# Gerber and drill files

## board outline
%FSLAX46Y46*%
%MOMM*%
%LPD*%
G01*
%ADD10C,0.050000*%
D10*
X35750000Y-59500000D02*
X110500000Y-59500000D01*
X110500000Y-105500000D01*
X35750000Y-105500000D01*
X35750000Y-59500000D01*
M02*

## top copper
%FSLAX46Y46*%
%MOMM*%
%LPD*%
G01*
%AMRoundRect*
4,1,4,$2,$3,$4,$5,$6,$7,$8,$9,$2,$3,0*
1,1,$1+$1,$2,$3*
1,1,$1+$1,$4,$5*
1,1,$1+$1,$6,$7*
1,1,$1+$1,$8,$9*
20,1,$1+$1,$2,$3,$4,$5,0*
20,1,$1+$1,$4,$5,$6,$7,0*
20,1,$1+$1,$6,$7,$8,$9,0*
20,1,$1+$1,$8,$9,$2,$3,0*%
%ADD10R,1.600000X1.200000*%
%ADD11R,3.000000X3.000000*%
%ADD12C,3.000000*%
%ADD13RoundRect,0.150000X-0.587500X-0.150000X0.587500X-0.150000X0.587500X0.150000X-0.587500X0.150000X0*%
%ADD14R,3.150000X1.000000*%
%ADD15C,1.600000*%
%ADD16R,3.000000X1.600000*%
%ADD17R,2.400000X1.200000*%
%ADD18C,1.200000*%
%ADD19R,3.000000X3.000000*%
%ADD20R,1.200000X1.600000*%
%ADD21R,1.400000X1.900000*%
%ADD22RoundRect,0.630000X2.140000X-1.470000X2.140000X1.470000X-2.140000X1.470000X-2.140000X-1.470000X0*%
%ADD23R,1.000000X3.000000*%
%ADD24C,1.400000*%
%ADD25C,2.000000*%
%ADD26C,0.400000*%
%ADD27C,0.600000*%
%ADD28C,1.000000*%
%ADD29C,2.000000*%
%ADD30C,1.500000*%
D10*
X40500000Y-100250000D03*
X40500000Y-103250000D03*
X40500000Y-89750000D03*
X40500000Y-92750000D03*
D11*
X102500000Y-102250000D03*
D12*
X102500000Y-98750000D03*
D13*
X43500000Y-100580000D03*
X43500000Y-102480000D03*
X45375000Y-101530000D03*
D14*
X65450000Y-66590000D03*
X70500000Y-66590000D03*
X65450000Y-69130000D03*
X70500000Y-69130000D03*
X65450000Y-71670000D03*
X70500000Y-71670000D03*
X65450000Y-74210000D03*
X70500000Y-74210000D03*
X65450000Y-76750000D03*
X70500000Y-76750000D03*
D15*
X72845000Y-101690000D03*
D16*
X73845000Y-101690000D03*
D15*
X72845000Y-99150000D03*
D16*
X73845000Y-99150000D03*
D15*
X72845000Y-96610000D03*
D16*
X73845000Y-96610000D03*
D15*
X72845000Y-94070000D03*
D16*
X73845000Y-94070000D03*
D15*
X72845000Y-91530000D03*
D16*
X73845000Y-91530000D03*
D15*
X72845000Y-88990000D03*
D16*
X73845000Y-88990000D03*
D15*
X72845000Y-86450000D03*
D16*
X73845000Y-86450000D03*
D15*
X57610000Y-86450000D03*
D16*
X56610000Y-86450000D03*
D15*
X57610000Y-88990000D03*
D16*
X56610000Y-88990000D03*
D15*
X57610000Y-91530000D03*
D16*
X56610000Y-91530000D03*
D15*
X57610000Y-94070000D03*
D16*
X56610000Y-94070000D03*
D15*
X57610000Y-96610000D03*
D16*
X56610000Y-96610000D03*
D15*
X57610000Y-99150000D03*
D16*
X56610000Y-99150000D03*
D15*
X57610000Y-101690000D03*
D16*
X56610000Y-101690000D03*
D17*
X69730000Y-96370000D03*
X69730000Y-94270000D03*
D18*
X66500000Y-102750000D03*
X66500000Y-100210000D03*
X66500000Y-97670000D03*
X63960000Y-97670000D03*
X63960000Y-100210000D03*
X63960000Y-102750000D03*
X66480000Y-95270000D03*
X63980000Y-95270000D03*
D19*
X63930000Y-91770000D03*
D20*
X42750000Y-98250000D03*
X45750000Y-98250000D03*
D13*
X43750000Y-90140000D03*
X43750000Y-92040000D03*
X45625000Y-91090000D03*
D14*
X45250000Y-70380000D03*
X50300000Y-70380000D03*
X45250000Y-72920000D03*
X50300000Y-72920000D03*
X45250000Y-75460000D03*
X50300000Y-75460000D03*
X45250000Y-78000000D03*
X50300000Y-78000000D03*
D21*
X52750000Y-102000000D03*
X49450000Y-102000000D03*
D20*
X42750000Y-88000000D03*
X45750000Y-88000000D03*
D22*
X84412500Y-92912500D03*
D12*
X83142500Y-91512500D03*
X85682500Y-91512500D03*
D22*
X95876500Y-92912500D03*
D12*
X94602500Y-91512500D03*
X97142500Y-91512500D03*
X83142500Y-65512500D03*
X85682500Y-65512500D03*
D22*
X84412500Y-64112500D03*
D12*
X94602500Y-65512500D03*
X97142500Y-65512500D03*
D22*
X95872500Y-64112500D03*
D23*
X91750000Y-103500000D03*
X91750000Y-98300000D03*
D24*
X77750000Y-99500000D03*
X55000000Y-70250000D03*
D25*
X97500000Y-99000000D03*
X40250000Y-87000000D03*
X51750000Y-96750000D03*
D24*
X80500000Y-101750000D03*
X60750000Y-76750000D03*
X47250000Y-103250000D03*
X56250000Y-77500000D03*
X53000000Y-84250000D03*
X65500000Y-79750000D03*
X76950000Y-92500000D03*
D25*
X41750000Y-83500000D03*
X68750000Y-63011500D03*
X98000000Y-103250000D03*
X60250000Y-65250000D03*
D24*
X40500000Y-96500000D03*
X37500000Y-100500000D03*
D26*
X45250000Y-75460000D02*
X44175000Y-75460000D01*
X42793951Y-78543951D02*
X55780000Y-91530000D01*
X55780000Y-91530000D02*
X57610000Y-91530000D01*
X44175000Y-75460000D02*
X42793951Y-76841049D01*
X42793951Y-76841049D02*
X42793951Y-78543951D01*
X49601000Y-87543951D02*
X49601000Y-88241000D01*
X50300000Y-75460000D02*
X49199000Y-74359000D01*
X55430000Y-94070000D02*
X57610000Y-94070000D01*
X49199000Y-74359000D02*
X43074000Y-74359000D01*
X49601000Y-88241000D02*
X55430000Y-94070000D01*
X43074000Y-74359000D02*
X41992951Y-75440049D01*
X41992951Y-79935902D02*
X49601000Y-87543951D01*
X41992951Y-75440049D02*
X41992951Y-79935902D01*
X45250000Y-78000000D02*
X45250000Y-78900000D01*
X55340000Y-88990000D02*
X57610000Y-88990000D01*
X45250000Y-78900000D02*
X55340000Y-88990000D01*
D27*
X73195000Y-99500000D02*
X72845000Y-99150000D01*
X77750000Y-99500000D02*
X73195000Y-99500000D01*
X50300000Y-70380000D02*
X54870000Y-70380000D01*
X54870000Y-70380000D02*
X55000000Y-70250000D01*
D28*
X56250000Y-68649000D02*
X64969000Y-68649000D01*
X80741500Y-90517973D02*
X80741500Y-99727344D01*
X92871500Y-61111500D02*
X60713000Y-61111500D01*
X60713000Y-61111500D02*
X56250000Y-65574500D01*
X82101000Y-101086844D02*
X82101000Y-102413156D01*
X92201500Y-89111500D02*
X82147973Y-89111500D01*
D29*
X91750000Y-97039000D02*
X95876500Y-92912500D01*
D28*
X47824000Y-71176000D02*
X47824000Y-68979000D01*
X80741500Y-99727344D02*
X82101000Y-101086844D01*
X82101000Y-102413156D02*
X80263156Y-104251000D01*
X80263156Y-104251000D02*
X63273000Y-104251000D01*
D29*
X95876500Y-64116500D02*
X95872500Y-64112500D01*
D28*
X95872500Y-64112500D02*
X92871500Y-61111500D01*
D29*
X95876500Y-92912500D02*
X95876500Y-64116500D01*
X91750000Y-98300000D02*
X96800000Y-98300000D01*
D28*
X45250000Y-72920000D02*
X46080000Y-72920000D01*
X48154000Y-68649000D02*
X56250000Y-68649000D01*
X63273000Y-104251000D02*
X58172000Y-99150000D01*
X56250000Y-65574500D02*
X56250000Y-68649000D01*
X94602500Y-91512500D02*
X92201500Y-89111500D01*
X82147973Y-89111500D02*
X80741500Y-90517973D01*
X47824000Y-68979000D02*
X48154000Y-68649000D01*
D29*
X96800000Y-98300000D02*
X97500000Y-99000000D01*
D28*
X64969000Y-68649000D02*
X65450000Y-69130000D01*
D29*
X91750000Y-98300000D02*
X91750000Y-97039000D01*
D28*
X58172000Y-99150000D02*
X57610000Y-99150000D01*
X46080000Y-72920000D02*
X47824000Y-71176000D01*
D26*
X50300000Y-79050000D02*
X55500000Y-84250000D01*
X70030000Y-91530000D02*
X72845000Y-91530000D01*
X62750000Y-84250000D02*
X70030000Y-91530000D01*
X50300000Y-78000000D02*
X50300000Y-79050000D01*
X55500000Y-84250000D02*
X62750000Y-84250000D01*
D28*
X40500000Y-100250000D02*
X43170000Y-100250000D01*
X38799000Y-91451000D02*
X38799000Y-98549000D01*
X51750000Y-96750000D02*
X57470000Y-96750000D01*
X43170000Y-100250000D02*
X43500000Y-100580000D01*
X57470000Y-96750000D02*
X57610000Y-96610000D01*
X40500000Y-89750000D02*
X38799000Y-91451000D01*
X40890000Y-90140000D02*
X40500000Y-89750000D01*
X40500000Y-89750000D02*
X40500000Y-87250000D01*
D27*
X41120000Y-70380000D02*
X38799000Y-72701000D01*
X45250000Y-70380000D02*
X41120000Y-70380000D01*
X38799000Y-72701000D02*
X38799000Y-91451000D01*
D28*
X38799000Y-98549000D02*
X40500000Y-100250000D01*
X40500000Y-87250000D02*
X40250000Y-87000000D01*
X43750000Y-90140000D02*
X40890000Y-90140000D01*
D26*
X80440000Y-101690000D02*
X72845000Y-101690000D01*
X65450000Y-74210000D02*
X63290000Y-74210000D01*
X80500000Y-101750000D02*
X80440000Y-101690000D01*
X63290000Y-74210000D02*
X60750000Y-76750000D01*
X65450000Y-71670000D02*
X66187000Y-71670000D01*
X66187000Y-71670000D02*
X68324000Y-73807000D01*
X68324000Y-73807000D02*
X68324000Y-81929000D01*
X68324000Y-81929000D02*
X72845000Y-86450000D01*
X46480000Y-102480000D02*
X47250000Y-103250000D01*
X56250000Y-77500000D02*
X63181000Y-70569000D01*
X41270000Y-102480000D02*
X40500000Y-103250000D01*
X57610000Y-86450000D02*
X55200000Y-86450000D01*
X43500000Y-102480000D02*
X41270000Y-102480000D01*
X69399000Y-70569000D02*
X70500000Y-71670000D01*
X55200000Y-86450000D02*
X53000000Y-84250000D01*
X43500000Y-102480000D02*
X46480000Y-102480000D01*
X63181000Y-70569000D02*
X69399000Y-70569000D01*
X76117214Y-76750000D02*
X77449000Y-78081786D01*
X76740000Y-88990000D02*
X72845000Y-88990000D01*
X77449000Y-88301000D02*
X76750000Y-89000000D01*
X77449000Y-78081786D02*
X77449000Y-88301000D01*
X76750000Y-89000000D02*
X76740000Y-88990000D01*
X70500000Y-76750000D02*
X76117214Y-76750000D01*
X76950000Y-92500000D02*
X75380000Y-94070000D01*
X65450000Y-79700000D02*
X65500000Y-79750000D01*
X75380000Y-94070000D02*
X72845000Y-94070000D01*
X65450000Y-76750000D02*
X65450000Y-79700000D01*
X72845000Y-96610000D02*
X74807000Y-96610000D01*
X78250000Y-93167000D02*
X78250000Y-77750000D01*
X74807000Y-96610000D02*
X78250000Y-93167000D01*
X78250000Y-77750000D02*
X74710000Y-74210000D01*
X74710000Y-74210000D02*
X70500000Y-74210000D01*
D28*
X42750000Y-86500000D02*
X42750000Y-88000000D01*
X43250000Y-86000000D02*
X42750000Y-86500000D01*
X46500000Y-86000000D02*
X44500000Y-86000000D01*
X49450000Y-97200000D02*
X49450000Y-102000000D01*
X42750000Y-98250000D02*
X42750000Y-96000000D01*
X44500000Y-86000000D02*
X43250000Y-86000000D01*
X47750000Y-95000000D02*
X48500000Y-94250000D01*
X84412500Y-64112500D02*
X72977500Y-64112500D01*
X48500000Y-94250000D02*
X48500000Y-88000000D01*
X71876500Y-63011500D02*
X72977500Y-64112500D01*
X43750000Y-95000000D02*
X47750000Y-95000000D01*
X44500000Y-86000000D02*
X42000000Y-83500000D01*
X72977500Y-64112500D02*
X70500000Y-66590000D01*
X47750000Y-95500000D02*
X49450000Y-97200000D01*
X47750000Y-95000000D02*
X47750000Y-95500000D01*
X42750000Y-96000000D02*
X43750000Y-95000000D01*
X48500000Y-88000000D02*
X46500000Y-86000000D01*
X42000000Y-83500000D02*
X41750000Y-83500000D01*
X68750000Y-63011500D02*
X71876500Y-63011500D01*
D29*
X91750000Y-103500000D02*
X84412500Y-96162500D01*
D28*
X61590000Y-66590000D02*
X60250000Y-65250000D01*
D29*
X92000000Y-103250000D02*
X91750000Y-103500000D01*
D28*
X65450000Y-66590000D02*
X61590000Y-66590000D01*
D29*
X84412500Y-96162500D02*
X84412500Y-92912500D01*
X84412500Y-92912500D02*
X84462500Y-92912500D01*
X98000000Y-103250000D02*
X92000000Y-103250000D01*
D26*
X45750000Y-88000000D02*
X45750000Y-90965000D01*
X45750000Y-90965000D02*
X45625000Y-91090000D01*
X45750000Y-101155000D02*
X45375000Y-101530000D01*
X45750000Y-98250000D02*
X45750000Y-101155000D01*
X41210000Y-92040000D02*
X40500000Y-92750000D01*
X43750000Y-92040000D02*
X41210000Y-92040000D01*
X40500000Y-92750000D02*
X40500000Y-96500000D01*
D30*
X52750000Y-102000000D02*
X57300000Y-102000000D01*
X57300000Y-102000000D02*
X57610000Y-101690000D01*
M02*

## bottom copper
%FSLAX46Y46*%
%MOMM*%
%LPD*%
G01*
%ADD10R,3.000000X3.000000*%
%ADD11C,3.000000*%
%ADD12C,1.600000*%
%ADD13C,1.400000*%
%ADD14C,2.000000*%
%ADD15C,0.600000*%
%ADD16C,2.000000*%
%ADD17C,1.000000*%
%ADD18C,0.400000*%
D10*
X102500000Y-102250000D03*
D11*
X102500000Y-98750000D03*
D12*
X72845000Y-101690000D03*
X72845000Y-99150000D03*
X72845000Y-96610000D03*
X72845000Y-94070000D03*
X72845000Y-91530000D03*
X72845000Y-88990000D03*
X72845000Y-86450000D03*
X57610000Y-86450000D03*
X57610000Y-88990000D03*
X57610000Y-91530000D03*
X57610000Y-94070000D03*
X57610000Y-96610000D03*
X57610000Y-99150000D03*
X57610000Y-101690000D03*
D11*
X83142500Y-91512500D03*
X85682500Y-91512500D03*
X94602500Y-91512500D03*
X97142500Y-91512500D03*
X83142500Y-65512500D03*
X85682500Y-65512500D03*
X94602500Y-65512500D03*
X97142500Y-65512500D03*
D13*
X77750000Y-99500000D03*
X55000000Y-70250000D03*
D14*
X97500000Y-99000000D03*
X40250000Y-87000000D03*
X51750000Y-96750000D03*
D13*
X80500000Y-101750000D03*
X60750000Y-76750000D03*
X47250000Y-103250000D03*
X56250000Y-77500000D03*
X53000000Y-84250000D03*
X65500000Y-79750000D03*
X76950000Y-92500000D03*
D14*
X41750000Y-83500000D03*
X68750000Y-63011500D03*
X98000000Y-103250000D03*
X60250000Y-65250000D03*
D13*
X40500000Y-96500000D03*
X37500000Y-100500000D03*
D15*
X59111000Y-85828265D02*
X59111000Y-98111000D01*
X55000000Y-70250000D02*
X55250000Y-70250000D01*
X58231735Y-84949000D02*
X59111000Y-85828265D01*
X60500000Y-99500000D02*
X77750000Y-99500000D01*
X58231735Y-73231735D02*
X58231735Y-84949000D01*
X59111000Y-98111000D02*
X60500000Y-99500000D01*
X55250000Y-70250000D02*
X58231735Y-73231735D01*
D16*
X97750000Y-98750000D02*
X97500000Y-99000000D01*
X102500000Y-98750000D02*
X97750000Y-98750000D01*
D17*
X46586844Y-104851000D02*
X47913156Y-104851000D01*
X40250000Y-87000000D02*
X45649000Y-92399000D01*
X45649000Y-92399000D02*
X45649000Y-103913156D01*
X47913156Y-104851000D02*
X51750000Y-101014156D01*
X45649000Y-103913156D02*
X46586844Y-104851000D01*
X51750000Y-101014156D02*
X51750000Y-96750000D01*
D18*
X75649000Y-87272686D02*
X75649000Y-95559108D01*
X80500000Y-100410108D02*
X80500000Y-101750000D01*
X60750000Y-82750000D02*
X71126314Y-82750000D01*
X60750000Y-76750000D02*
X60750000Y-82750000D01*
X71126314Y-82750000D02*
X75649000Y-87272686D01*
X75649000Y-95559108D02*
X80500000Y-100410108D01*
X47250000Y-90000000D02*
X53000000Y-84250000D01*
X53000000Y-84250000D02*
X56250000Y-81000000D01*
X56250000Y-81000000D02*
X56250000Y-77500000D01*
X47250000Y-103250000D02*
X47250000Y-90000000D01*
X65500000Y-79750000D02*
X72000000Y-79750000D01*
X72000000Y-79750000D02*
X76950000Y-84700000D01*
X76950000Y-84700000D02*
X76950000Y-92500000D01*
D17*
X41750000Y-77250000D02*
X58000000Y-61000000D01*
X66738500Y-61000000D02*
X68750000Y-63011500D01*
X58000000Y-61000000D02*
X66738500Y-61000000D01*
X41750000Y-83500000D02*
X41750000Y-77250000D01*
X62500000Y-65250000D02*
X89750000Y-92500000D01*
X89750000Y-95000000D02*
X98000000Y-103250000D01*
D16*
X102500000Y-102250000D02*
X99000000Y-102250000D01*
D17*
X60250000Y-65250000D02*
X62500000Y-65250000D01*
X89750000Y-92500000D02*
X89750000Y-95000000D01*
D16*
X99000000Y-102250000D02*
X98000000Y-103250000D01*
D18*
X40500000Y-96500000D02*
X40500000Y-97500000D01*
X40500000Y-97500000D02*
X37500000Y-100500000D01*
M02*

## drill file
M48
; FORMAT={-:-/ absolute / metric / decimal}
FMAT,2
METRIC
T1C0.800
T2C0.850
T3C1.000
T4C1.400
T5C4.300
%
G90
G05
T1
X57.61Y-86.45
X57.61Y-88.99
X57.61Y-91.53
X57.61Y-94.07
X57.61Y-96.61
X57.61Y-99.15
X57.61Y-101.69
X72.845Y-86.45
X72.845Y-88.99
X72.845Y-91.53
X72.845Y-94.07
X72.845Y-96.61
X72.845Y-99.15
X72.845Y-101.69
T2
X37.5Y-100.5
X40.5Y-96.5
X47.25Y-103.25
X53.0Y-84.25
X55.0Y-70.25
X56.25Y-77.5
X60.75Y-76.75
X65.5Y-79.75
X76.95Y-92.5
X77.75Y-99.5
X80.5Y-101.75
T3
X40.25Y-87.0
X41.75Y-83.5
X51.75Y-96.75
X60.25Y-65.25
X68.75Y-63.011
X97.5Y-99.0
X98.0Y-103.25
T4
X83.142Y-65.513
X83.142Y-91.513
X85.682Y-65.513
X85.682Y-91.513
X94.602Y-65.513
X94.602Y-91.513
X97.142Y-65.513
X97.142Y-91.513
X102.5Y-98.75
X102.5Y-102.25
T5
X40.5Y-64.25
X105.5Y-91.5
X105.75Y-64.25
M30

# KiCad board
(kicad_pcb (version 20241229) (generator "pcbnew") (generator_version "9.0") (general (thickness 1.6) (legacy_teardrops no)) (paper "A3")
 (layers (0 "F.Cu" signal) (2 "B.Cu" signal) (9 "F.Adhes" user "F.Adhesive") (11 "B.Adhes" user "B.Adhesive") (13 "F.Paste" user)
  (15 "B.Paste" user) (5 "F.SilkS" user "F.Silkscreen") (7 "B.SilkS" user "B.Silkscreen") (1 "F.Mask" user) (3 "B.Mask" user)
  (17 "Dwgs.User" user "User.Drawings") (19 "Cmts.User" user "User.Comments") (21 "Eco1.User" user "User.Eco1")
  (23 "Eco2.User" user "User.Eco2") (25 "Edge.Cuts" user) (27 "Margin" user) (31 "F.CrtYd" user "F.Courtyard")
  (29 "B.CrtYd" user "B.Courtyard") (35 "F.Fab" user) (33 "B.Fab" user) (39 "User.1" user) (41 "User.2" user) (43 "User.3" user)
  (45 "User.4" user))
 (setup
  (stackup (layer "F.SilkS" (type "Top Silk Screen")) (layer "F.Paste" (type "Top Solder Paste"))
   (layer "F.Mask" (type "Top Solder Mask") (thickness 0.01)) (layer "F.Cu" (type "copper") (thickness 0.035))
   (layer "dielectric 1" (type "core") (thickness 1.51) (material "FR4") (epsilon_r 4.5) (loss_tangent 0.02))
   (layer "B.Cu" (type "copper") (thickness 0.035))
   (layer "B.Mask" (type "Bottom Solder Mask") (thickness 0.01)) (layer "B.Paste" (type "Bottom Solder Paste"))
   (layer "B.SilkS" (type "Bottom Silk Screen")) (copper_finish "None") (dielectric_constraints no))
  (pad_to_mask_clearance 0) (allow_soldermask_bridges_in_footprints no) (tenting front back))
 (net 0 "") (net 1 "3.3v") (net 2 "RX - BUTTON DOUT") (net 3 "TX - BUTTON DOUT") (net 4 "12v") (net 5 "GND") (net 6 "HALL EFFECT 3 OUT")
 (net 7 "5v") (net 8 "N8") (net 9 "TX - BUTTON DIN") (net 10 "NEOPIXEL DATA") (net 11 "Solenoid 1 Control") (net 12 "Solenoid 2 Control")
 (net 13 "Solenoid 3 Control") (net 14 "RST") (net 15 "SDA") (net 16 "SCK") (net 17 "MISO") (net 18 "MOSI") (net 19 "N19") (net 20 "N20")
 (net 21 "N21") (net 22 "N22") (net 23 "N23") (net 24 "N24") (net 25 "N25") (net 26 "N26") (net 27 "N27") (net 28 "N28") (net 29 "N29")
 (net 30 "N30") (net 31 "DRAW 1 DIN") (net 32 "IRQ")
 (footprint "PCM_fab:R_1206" (layer "F.Cu") (at 40.5 101.75 -90)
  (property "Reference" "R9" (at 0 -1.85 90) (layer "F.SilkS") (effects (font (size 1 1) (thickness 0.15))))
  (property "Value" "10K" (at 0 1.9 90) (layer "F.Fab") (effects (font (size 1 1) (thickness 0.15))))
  (pad "1" smd rect (at -1.5 0 270) (size 1.2 1.6) (layers "F.Cu" "F.Mask" "F.Paste") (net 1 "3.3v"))
  (pad "2" smd rect (at 1.5 0 270) (size 1.2 1.6) (layers "F.Cu" "F.Mask" "F.Paste") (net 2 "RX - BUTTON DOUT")))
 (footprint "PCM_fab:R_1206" (layer "F.Cu") (at 40.5 91.25 -90)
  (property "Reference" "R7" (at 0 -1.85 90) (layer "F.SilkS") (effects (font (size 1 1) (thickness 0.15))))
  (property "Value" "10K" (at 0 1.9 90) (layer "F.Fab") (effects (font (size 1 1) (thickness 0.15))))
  (pad "1" smd rect (at -1.5 0 270) (size 1.2 1.6) (layers "F.Cu" "F.Mask" "F.Paste") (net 1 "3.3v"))
  (pad "2" smd rect (at 1.5 0 270) (size 1.2 1.6) (layers "F.Cu" "F.Mask" "F.Paste") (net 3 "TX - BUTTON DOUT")))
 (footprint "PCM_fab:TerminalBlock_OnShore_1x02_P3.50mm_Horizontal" (layer "F.Cu") (at 102.5 102.25 90)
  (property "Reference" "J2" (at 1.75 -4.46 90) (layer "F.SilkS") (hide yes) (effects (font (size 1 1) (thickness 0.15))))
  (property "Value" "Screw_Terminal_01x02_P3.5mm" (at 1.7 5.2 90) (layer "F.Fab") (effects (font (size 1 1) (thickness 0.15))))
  (pad "1" thru_hole rect (at 0 0 90) (size 3 3) (drill 1.4) (layers "*.Cu" "*.Mask") (remove_unused_layers no) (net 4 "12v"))
  (pad "2" thru_hole circle (at 3.5 0 90) (size 3 3) (drill 1.4) (layers "*.Cu" "*.Mask") (remove_unused_layers no) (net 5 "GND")))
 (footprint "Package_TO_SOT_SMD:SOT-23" (layer "F.Cu") (at 44.4375 101.53)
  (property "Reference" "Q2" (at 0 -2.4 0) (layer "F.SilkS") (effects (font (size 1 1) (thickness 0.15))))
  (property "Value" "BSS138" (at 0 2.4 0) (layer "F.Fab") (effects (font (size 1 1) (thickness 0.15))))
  (pad "1" smd roundrect (at -0.9375 -0.95) (size 1.475 0.6) (layers "F.Cu" "F.Mask" "F.Paste") (roundrect_rratio 0.25) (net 1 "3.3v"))
  (pad "2" smd roundrect (at -0.9375 0.95) (size 1.475 0.6) (layers "F.Cu" "F.Mask" "F.Paste") (roundrect_rratio 0.25)
   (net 2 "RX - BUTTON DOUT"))
  (pad "3" smd roundrect (at 0.9375 0) (size 1.475 0.6) (layers "F.Cu" "F.Mask" "F.Paste") (roundrect_rratio 0.25)
   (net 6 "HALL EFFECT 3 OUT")))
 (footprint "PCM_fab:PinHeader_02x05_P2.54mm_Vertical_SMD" (layer "F.Cu") (at 67.975 71.67)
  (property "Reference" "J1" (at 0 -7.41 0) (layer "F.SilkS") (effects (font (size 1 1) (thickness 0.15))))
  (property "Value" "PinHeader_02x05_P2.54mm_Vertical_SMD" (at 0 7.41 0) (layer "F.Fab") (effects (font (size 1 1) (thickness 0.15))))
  (pad "1" smd rect (at -2.525 -5.08) (size 3.15 1) (layers "F.Cu" "F.Mask" "F.Paste") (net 4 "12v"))
  (pad "2" smd rect (at 2.525 -5.08) (size 3.15 1) (layers "F.Cu" "F.Mask" "F.Paste") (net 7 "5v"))
  (pad "3" smd rect (at -2.525 -2.54) (size 3.15 1) (layers "F.Cu" "F.Mask" "F.Paste") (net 5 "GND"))
  (pad "4" smd rect (at 2.525 -2.54) (size 3.15 1) (layers "F.Cu" "F.Mask" "F.Paste") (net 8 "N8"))
  (pad "5" smd rect (at -2.525 0) (size 3.15 1) (layers "F.Cu" "F.Mask" "F.Paste") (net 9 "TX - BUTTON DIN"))
  (pad "6" smd rect (at 2.525 0) (size 3.15 1) (layers "F.Cu" "F.Mask" "F.Paste") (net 2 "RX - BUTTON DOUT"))
  (pad "7" smd rect (at -2.525 2.54) (size 3.15 1) (layers "F.Cu" "F.Mask" "F.Paste") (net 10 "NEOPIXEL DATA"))
  (pad "8" smd rect (at 2.525 2.54) (size 3.15 1) (layers "F.Cu" "F.Mask" "F.Paste") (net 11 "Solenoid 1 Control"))
  (pad "9" smd rect (at -2.525 5.08) (size 3.15 1) (layers "F.Cu" "F.Mask" "F.Paste") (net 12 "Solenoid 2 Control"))
  (pad "10" smd rect (at 2.525 5.08) (size 3.15 1) (layers "F.Cu" "F.Mask" "F.Paste") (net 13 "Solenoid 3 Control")))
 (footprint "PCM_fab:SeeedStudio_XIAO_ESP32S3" (layer "F.Cu") (at 65.23 94.07 180)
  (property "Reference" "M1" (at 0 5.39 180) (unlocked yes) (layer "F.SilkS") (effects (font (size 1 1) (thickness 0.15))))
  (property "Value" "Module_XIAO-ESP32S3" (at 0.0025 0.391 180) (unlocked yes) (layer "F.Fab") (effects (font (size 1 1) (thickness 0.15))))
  (pad "1" thru_hole circle (at -7.615 -7.62 180) (size 1.6 1.6) (drill 0.8) (layers "*.Cu" "*.Mask") (remove_unused_layers no)
   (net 10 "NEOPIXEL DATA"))
  (pad "1" smd rect (at -7.615 -7.62 180) (size 3 1.6) (drill (offset -1 0)) (layers "F.Cu" "F.Mask" "F.Paste") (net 10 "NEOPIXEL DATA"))
  (pad "2" thru_hole circle (at -7.615 -5.08 180) (size 1.6 1.6) (drill 0.8) (layers "*.Cu" "*.Mask") (remove_unused_layers no)
   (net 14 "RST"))
  (pad "2" smd rect (at -7.615 -5.08 180) (size 3 1.6) (drill (offset -1 0)) (layers "F.Cu" "F.Mask" "F.Paste") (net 14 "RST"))
  (pad "3" thru_hole circle (at -7.615 -2.54 180) (size 1.6 1.6) (drill 0.8) (layers "*.Cu" "*.Mask") (remove_unused_layers no)
   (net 11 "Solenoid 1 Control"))
  (pad "3" smd rect (at -7.615 -2.54 180) (size 3 1.6) (drill (offset -1 0)) (layers "F.Cu" "F.Mask" "F.Paste")
   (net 11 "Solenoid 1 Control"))
  (pad "4" thru_hole circle (at -7.615 0 180) (size 1.6 1.6) (drill 0.8) (layers "*.Cu" "*.Mask") (remove_unused_layers no)
   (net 12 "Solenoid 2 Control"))
  (pad "4" smd rect (at -7.615 0 180) (size 3 1.6) (drill (offset -1 0)) (layers "F.Cu" "F.Mask" "F.Paste") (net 12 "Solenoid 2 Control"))
  (pad "5" thru_hole circle (at -7.615 2.54 180) (size 1.6 1.6) (drill 0.8) (layers "*.Cu" "*.Mask") (remove_unused_layers no)
   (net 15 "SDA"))
  (pad "5" smd rect (at -7.615 2.54 180) (size 3 1.6) (drill (offset -1 0)) (layers "F.Cu" "F.Mask" "F.Paste") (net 15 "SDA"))
  (pad "6" thru_hole circle (at -7.615 5.08 180) (size 1.6 1.6) (drill 0.8) (layers "*.Cu" "*.Mask") (remove_unused_layers no)
   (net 13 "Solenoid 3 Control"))
  (pad "6" smd rect (at -7.615 5.08 180) (size 3 1.6) (drill (offset -1 0)) (layers "F.Cu" "F.Mask" "F.Paste") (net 13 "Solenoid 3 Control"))
  (pad "7" thru_hole circle (at -7.615 7.62 180) (size 1.6 1.6) (drill 0.8) (layers "*.Cu" "*.Mask") (remove_unused_layers no)
   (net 9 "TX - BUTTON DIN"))
  (pad "7" smd rect (at -7.615 7.62 180) (size 3 1.6) (drill (offset -1 0)) (layers "F.Cu" "F.Mask" "F.Paste") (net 9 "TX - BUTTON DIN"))
  (pad "8" thru_hole circle (at 7.62 7.62 180) (size 1.6 1.6) (drill 0.8) (layers "*.Cu" "*.Mask") (remove_unused_layers no)
   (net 2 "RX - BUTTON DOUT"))
  (pad "8" smd rect (at 7.62 7.62 180) (size 3 1.6) (drill (offset 1 0)) (layers "F.Cu" "F.Mask" "F.Paste") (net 2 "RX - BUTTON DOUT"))
  (pad "9" thru_hole circle (at 7.62 5.08 180) (size 1.6 1.6) (drill 0.8) (layers "*.Cu" "*.Mask") (remove_unused_layers no) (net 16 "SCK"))
  (pad "9" smd rect (at 7.62 5.08 180) (size 3 1.6) (drill (offset 1 0)) (layers "F.Cu" "F.Mask" "F.Paste") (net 16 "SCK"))
  (pad "10" thru_hole circle (at 7.62 2.54 180) (size 1.6 1.6) (drill 0.8) (layers "*.Cu" "*.Mask") (remove_unused_layers no)
   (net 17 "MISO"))
  (pad "10" smd rect (at 7.62 2.54 180) (size 3 1.6) (drill (offset 1 0)) (layers "F.Cu" "F.Mask" "F.Paste") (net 17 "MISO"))
  (pad "11" thru_hole circle (at 7.62 0 180) (size 1.6 1.6) (drill 0.8) (layers "*.Cu" "*.Mask") (remove_unused_layers no) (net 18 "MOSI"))
  (pad "11" smd rect (at 7.62 0 180) (size 3 1.6) (drill (offset 1 0)) (layers "F.Cu" "F.Mask" "F.Paste") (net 18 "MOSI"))
  (pad "12" thru_hole circle (at 7.62 -2.54 180) (size 1.6 1.6) (drill 0.8) (layers "*.Cu" "*.Mask") (remove_unused_layers no)
   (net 1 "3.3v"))
  (pad "12" smd rect (at 7.62 -2.54 180) (size 3 1.6) (drill (offset 1 0)) (layers "F.Cu" "F.Mask" "F.Paste") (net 1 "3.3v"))
  (pad "13" thru_hole circle (at 7.62 -5.08 180) (size 1.6 1.6) (drill 0.8) (layers "*.Cu" "*.Mask") (remove_unused_layers no) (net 5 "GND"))
  (pad "13" smd rect (at 7.62 -5.08 180) (size 3 1.6) (drill (offset 1 0)) (layers "F.Cu" "F.Mask" "F.Paste") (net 5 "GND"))
  (pad "14" thru_hole circle (at 7.62 -7.62 180) (size 1.6 1.6) (drill 0.8) (layers "*.Cu" "*.Mask") (remove_unused_layers no)
   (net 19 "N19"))
  (pad "14" smd rect (at 7.62 -7.62 180) (size 3 1.6) (drill (offset 1 0)) (layers "F.Cu" "F.Mask" "F.Paste") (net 19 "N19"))
  (pad "15" smd rect (at -4.5 -2.3 180) (size 2.4 1.2) (layers "F.Cu" "F.Mask" "F.Paste") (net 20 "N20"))
  (pad "16" smd rect (at -4.5 -0.2 180) (size 2.4 1.2) (layers "F.Cu" "F.Mask" "F.Paste") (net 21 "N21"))
  (pad "17" smd circle (at -1.27 -8.68 180) (size 1.2 1.2) (layers "F.Cu" "F.Mask" "F.Paste") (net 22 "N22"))
  (pad "18" smd circle (at -1.27 -6.14 180) (size 1.2 1.2) (layers "F.Cu" "F.Mask" "F.Paste") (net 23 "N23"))
  (pad "19" smd circle (at -1.27 -3.6 180) (size 1.2 1.2) (layers "F.Cu" "F.Mask" "F.Paste") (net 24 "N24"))
  (pad "20" smd circle (at 1.27 -3.6 180) (size 1.2 1.2) (layers "F.Cu" "F.Mask" "F.Paste") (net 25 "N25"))
  (pad "21" smd circle (at 1.27 -6.14 180) (size 1.2 1.2) (layers "F.Cu" "F.Mask" "F.Paste") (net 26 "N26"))
  (pad "22" smd circle (at 1.27 -8.68 180) (size 1.2 1.2) (layers "F.Cu" "F.Mask" "F.Paste") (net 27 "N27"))
  (pad "23" smd circle (at -1.25 -1.2 180) (size 1.2 1.2) (layers "F.Cu" "F.Mask" "F.Paste") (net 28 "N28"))
  (pad "24" smd circle (at 1.25 -1.2 180) (size 1.2 1.2) (layers "F.Cu" "F.Mask" "F.Paste") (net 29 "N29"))
  (pad "25" smd rect (at 1.3 2.3 180) (size 3 3) (layers "F.Cu" "F.Mask" "F.Paste") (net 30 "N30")))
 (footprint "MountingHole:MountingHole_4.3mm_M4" (layer "F.Cu") (at 105.75 64.25)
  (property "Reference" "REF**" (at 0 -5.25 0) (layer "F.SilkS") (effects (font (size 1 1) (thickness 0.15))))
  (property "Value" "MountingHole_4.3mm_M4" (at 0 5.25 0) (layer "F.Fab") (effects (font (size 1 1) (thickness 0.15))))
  (pad "" np_thru_hole circle (at 0 0) (size 4.3 4.3) (drill 4.3) (layers "*.Cu" "*.Mask")))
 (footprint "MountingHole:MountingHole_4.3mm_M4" (layer "F.Cu") (at 40.5 64.25)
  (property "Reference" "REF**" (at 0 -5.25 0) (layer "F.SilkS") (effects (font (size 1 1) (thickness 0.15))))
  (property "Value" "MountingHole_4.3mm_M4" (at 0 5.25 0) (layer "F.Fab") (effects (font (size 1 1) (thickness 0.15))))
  (pad "" np_thru_hole circle (at 0 0) (size 4.3 4.3) (drill 4.3) (layers "*.Cu" "*.Mask")))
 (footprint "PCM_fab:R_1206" (layer "F.Cu") (at 44.25 98.25)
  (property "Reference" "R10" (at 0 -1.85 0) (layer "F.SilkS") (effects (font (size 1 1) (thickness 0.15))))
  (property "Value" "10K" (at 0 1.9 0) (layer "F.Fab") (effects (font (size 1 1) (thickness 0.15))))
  (pad "1" smd rect (at -1.5 0) (size 1.2 1.6) (layers "F.Cu" "F.Mask" "F.Paste") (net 7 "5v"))
  (pad "2" smd rect (at 1.5 0) (size 1.2 1.6) (layers "F.Cu" "F.Mask" "F.Paste") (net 6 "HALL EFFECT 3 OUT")))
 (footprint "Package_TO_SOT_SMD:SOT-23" (layer "F.Cu") (at 44.6875 91.09)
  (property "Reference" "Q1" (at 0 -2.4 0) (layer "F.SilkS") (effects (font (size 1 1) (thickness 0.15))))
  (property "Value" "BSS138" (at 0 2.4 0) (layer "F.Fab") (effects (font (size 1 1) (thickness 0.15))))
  (pad "1" smd roundrect (at -0.9375 -0.95) (size 1.475 0.6) (layers "F.Cu" "F.Mask" "F.Paste") (roundrect_rratio 0.25) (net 1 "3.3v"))
  (pad "2" smd roundrect (at -0.9375 0.95) (size 1.475 0.6) (layers "F.Cu" "F.Mask" "F.Paste") (roundrect_rratio 0.25)
   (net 3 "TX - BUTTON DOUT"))
  (pad "3" smd roundrect (at 0.9375 0) (size 1.475 0.6) (layers "F.Cu" "F.Mask" "F.Paste") (roundrect_rratio 0.25) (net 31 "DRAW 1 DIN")))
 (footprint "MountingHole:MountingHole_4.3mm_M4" (layer "F.Cu") (at 105.5 91.5)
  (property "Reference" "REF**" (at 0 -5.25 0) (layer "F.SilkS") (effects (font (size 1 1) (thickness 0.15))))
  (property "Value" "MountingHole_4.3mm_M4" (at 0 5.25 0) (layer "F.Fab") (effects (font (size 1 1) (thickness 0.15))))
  (pad "" np_thru_hole circle (at 0 0) (size 4.3 4.3) (drill 4.3) (layers "*.Cu" "*.Mask")))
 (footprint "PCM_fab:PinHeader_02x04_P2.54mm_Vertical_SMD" (layer "F.Cu") (at 47.775 74.19)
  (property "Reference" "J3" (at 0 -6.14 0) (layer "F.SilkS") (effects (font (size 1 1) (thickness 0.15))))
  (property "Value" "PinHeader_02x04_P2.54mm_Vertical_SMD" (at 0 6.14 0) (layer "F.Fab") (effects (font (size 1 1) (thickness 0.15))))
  (pad "1" smd rect (at -2.525 -3.81) (size 3.15 1) (layers "F.Cu" "F.Mask" "F.Paste") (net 1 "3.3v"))
  (pad "2" smd rect (at 2.525 -3.81) (size 3.15 1) (layers "F.Cu" "F.Mask" "F.Paste") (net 14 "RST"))
  (pad "3" smd rect (at -2.525 -1.27) (size 3.15 1) (layers "F.Cu" "F.Mask" "F.Paste") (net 5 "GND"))
  (pad "4" smd rect (at 2.525 -1.27) (size 3.15 1) (layers "F.Cu" "F.Mask" "F.Paste") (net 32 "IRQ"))
  (pad "5" smd rect (at -2.525 1.27) (size 3.15 1) (layers "F.Cu" "F.Mask" "F.Paste") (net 17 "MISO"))
  (pad "6" smd rect (at 2.525 1.27) (size 3.15 1) (layers "F.Cu" "F.Mask" "F.Paste") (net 18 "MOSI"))
  (pad "7" smd rect (at -2.525 3.81) (size 3.15 1) (layers "F.Cu" "F.Mask" "F.Paste") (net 16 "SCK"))
  (pad "8" smd rect (at 2.525 3.81) (size 3.15 1) (layers "F.Cu" "F.Mask" "F.Paste") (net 15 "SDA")))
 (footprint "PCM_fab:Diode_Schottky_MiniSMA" (layer "F.Cu") (at 51.1 102 180)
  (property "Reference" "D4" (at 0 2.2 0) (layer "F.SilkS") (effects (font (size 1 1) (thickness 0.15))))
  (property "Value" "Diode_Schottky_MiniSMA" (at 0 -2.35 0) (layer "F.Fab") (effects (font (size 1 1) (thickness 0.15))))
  (pad "1" smd rect (at -1.65 0 180) (size 1.4 1.9) (layers "F.Cu" "F.Mask" "F.Paste") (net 19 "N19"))
  (pad "2" smd rect (at 1.65 0 180) (size 1.4 1.9) (layers "F.Cu" "F.Mask" "F.Paste") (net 7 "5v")))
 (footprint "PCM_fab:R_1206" (layer "F.Cu") (at 44.25 88)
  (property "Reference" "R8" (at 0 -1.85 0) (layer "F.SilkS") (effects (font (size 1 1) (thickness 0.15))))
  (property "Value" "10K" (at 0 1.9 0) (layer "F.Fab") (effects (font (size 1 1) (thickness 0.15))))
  (pad "1" smd rect (at -1.5 0) (size 1.2 1.6) (layers "F.Cu" "F.Mask" "F.Paste") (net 7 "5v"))
  (pad "2" smd rect (at 1.5 0) (size 1.2 1.6) (layers "F.Cu" "F.Mask" "F.Paste") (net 31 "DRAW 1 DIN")))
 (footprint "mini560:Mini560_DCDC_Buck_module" (layer "F.Cu") (at 90.1425 78.5125 90)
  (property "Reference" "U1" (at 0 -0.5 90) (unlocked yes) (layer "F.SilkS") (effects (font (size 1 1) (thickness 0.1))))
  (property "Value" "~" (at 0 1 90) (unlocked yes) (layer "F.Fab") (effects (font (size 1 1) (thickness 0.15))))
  (pad "1" smd roundrect (at -14.4 -5.73 90) (size 4.2 5.54) (layers "F.Cu" "F.Mask" "F.Paste") (roundrect_rratio 0.15) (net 4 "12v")
   (thermal_bridge_angle 45))
  (pad "1" thru_hole circle (at -13 -7 90) (size 3 3) (drill 1.4) (layers "*.Cu" "*.Mask") (remove_unused_layers no) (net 4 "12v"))
  (pad "1" thru_hole circle (at -13 -4.46 90) (size 3 3) (drill 1.4) (layers "*.Cu" "*.Mask") (remove_unused_layers no) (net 4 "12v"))
  (pad "2" smd roundrect (at -14.4 5.734 90) (size 4.2 5.54) (layers "F.Cu" "F.Mask" "F.Paste") (roundrect_rratio 0.15) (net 5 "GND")
   (thermal_bridge_angle 45))
  (pad "2" thru_hole circle (at -13 4.46 90) (size 3 3) (drill 1.4) (layers "*.Cu" "*.Mask") (remove_unused_layers no) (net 5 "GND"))
  (pad "2" thru_hole circle (at -13 7 90) (size 3 3) (drill 1.4) (layers "*.Cu" "*.Mask") (remove_unused_layers no) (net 5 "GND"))
  (pad "3" thru_hole circle (at 13 -7 90) (size 3 3) (drill 1.4) (layers "*.Cu" "*.Mask") (remove_unused_layers no) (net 7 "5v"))
  (pad "3" thru_hole circle (at 13 -4.46 90) (size 3 3) (drill 1.4) (layers "*.Cu" "*.Mask") (remove_unused_layers no) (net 7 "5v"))
  (pad "3" smd roundrect (at 14.4 -5.73 90) (size 4.2 5.54) (layers "F.Cu" "F.Mask" "F.Paste") (roundrect_rratio 0.15) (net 7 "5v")
   (thermal_bridge_angle 45))
  (pad "4" thru_hole circle (at 13 4.46 90) (size 3 3) (drill 1.4) (layers "*.Cu" "*.Mask") (remove_unused_layers no) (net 5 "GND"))
  (pad "4" thru_hole circle (at 13 7 90) (size 3 3) (drill 1.4) (layers "*.Cu" "*.Mask") (remove_unused_layers no) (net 5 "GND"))
  (pad "4" smd roundrect (at 14.4 5.73 90) (size 4.2 5.54) (layers "F.Cu" "F.Mask" "F.Paste") (roundrect_rratio 0.15) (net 5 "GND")
   (thermal_bridge_angle 45)))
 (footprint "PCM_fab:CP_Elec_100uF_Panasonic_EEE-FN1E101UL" (layer "F.Cu") (at 91.75 100.9 90)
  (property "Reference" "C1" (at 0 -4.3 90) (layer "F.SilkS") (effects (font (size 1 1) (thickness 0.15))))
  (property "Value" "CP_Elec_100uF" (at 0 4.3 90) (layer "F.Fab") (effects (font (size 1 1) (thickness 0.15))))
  (pad "1" smd rect (at -2.6 0 90) (size 3 1) (layers "F.Cu" "F.Mask" "F.Paste") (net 4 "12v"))
  (pad "2" smd rect (at 2.6 0 90) (size 3 1) (layers "F.Cu" "F.Mask" "F.Paste") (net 5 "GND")))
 (gr_rect (start 35.75 59.5) (end 110.5 105.5) (stroke (width 0.05) (type default)) (fill no) (layer "Edge.Cuts"))
 (segment (start 45.25 75.46) (end 44.175 75.46) (width 0.4) (layer "F.Cu") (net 17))
 (segment (start 42.793951 78.543951) (end 55.78 91.53) (width 0.4) (layer "F.Cu") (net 17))
 (segment (start 55.78 91.53) (end 57.61 91.53) (width 0.4) (layer "F.Cu") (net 17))
 (segment (start 44.175 75.46) (end 42.793951 76.841049) (width 0.4) (layer "F.Cu") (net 17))
 (segment (start 42.793951 76.841049) (end 42.793951 78.543951) (width 0.4) (layer "F.Cu") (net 17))
 (segment (start 49.601 87.543951) (end 49.601 88.241) (width 0.4) (layer "F.Cu") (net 18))
 (segment (start 50.3 75.46) (end 49.199 74.359) (width 0.4) (layer "F.Cu") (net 18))
 (segment (start 55.43 94.07) (end 57.61 94.07) (width 0.4) (layer "F.Cu") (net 18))
 (segment (start 49.199 74.359) (end 43.074 74.359) (width 0.4) (layer "F.Cu") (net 18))
 (segment (start 49.601 88.241) (end 55.43 94.07) (width 0.4) (layer "F.Cu") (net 18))
 (segment (start 43.074 74.359) (end 41.992951 75.440049) (width 0.4) (layer "F.Cu") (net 18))
 (segment (start 41.992951 79.935902) (end 49.601 87.543951) (width 0.4) (layer "F.Cu") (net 18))
 (segment (start 41.992951 75.440049) (end 41.992951 79.935902) (width 0.4) (layer "F.Cu") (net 18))
 (segment (start 45.25 78) (end 45.25 78.9) (width 0.4) (layer "F.Cu") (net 16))
 (segment (start 55.34 88.99) (end 57.61 88.99) (width 0.4) (layer "F.Cu") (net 16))
 (segment (start 45.25 78.9) (end 55.34 88.99) (width 0.4) (layer "F.Cu") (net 16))
 (segment (start 73.195 99.5) (end 72.845 99.15) (width 0.6) (layer "F.Cu") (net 14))
 (segment (start 77.75 99.5) (end 73.195 99.5) (width 0.6) (layer "F.Cu") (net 14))
 (segment (start 50.3 70.38) (end 54.87 70.38) (width 0.6) (layer "F.Cu") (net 14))
 (segment (start 54.87 70.38) (end 55 70.25) (width 0.6) (layer "F.Cu") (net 14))
 (via (at 77.75 99.5) (size 1.4) (drill 0.85) (layers "F.Cu" "B.Cu") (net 14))
 (via (at 55 70.25) (size 1.4) (drill 0.85) (layers "F.Cu" "B.Cu") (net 14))
 (segment (start 59.111 85.828265) (end 59.111 98.111) (width 0.6) (layer "B.Cu") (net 14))
 (segment (start 55 70.25) (end 55.25 70.25) (width 0.6) (layer "B.Cu") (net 14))
 (segment (start 58.231735 84.949) (end 59.111 85.828265) (width 0.6) (layer "B.Cu") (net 14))
 (segment (start 60.5 99.5) (end 77.75 99.5) (width 0.6) (layer "B.Cu") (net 14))
 (segment (start 58.231735 73.231735) (end 58.231735 84.949) (width 0.6) (layer "B.Cu") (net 14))
 (segment (start 59.111 98.111) (end 60.5 99.5) (width 0.6) (layer "B.Cu") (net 14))
 (segment (start 55.25 70.25) (end 58.231735 73.231735) (width 0.6) (layer "B.Cu") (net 14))
 (segment (start 56.25 68.649) (end 64.969 68.649) (width 1) (layer "F.Cu") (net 5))
 (segment (start 80.7415 90.517973) (end 80.7415 99.727344) (width 1) (layer "F.Cu") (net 5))
 (segment (start 92.8715 61.1115) (end 60.713 61.1115) (width 1) (layer "F.Cu") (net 5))
 (segment (start 60.713 61.1115) (end 56.25 65.5745) (width 1) (layer "F.Cu") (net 5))
 (segment (start 82.101 101.086844) (end 82.101 102.413156) (width 1) (layer "F.Cu") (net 5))
 (segment (start 92.2015 89.1115) (end 82.147973 89.1115) (width 1) (layer "F.Cu") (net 5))
 (segment (start 91.75 97.039) (end 95.8765 92.9125) (width 2) (layer "F.Cu") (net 5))
 (segment (start 47.824 71.176) (end 47.824 68.979) (width 1) (layer "F.Cu") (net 5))
 (segment (start 80.7415 99.727344) (end 82.101 101.086844) (width 1) (layer "F.Cu") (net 5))
 (segment (start 82.101 102.413156) (end 80.263156 104.251) (width 1) (layer "F.Cu") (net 5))
 (segment (start 80.263156 104.251) (end 63.273 104.251) (width 1) (layer "F.Cu") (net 5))
 (segment (start 95.8765 64.1165) (end 95.8725 64.1125) (width 2) (layer "F.Cu") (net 5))
 (segment (start 95.8725 64.1125) (end 92.8715 61.1115) (width 1) (layer "F.Cu") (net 5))
 (segment (start 95.8765 92.9125) (end 95.8765 64.1165) (width 2) (layer "F.Cu") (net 5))
 (segment (start 91.75 98.3) (end 96.8 98.3) (width 2) (layer "F.Cu") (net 5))
 (segment (start 45.25 72.92) (end 46.08 72.92) (width 1) (layer "F.Cu") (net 5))
 (segment (start 48.154 68.649) (end 56.25 68.649) (width 1) (layer "F.Cu") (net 5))
 (segment (start 63.273 104.251) (end 58.172 99.15) (width 1) (layer "F.Cu") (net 5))
 (segment (start 56.25 65.5745) (end 56.25 68.649) (width 1) (layer "F.Cu") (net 5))
 (segment (start 94.6025 91.5125) (end 92.2015 89.1115) (width 1) (layer "F.Cu") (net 5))
 (segment (start 82.147973 89.1115) (end 80.7415 90.517973) (width 1) (layer "F.Cu") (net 5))
 (segment (start 47.824 68.979) (end 48.154 68.649) (width 1) (layer "F.Cu") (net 5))
 (segment (start 96.8 98.3) (end 97.5 99) (width 2) (layer "F.Cu") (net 5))
 (segment (start 64.969 68.649) (end 65.45 69.13) (width 1) (layer "F.Cu") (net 5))
 (segment (start 91.75 98.3) (end 91.75 97.039) (width 2) (layer "F.Cu") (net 5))
 (segment (start 58.172 99.15) (end 57.61 99.15) (width 1) (layer "F.Cu") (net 5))
 (segment (start 46.08 72.92) (end 47.824 71.176) (width 1) (layer "F.Cu") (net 5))
 (via (at 97.5 99) (size 2) (drill 1) (layers "F.Cu" "B.Cu") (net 5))
 (segment (start 97.75 98.75) (end 97.5 99) (width 2) (layer "B.Cu") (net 5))
 (segment (start 102.5 98.75) (end 97.75 98.75) (width 2) (layer "B.Cu") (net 5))
 (segment (start 50.3 79.05) (end 55.5 84.25) (width 0.4) (layer "F.Cu") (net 15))
 (segment (start 70.03 91.53) (end 72.845 91.53) (width 0.4) (layer "F.Cu") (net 15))
 (segment (start 62.75 84.25) (end 70.03 91.53) (width 0.4) (layer "F.Cu") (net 15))
 (segment (start 50.3 78) (end 50.3 79.05) (width 0.4) (layer "F.Cu") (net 15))
 (segment (start 55.5 84.25) (end 62.75 84.25) (width 0.4) (layer "F.Cu") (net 15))
 (segment (start 40.5 100.25) (end 43.17 100.25) (width 1) (layer "F.Cu") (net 1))
 (segment (start 38.799 91.451) (end 38.799 98.549) (width 1) (layer "F.Cu") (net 1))
 (segment (start 51.75 96.75) (end 57.47 96.75) (width 1) (layer "F.Cu") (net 1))
 (segment (start 43.17 100.25) (end 43.5 100.58) (width 1) (layer "F.Cu") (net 1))
 (segment (start 57.47 96.75) (end 57.61 96.61) (width 1) (layer "F.Cu") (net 1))
 (segment (start 40.5 89.75) (end 38.799 91.451) (width 1) (layer "F.Cu") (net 1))
 (segment (start 40.89 90.14) (end 40.5 89.75) (width 1) (layer "F.Cu") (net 1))
 (segment (start 40.5 89.75) (end 40.5 87.25) (width 1) (layer "F.Cu") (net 1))
 (segment (start 41.12 70.38) (end 38.799 72.701) (width 0.6) (layer "F.Cu") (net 1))
 (segment (start 45.25 70.38) (end 41.12 70.38) (width 0.6) (layer "F.Cu") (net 1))
 (segment (start 38.799 72.701) (end 38.799 91.451) (width 0.6) (layer "F.Cu") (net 1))
 (segment (start 38.799 98.549) (end 40.5 100.25) (width 1) (layer "F.Cu") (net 1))
 (segment (start 40.5 87.25) (end 40.25 87) (width 1) (layer "F.Cu") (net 1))
 (segment (start 43.75 90.14) (end 40.89 90.14) (width 1) (layer "F.Cu") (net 1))
 (via (at 40.25 87) (size 2) (drill 1) (layers "F.Cu" "B.Cu") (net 1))
 (via (at 51.75 96.75) (size 2) (drill 1) (layers "F.Cu" "B.Cu") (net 1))
 (segment (start 46.586844 104.851) (end 47.913156 104.851) (width 1) (layer "B.Cu") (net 1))
 (segment (start 40.25 87) (end 45.649 92.399) (width 1) (layer "B.Cu") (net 1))
 (segment (start 45.649 92.399) (end 45.649 103.913156) (width 1) (layer "B.Cu") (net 1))
 (segment (start 47.913156 104.851) (end 51.75 101.014156) (width 1) (layer "B.Cu") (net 1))
 (segment (start 45.649 103.913156) (end 46.586844 104.851) (width 1) (layer "B.Cu") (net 1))
 (segment (start 51.75 101.014156) (end 51.75 96.75) (width 1) (layer "B.Cu") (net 1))
 (segment (start 80.44 101.69) (end 72.845 101.69) (width 0.4) (layer "F.Cu") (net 10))
 (segment (start 65.45 74.21) (end 63.29 74.21) (width 0.4) (layer "F.Cu") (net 10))
 (segment (start 80.5 101.75) (end 80.44 101.69) (width 0.4) (layer "F.Cu") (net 10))
 (segment (start 63.29 74.21) (end 60.75 76.75) (width 0.4) (layer "F.Cu") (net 10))
 (via (at 80.5 101.75) (size 1.4) (drill 0.85) (layers "F.Cu" "B.Cu") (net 10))
 (via (at 60.75 76.75) (size 1.4) (drill 0.85) (layers "F.Cu" "B.Cu") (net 10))
 (segment (start 75.649 87.272686) (end 75.649 95.559108) (width 0.4) (layer "B.Cu") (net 10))
 (segment (start 80.5 100.410108) (end 80.5 101.75) (width 0.4) (layer "B.Cu") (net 10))
 (segment (start 60.75 82.75) (end 71.126314 82.75) (width 0.4) (layer "B.Cu") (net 10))
 (segment (start 60.75 76.75) (end 60.75 82.75) (width 0.4) (layer "B.Cu") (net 10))
 (segment (start 71.126314 82.75) (end 75.649 87.272686) (width 0.4) (layer "B.Cu") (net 10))
 (segment (start 75.649 95.559108) (end 80.5 100.410108) (width 0.4) (layer "B.Cu") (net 10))
 (segment (start 65.45 71.67) (end 66.187 71.67) (width 0.4) (layer "F.Cu") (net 9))
 (segment (start 66.187 71.67) (end 68.324 73.807) (width 0.4) (layer "F.Cu") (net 9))
 (segment (start 68.324 73.807) (end 68.324 81.929) (width 0.4) (layer "F.Cu") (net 9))
 (segment (start 68.324 81.929) (end 72.845 86.45) (width 0.4) (layer "F.Cu") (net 9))
 (segment (start 46.48 102.48) (end 47.25 103.25) (width 0.4) (layer "F.Cu") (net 2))
 (segment (start 56.25 77.5) (end 63.181 70.569) (width 0.4) (layer "F.Cu") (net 2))
 (segment (start 41.27 102.48) (end 40.5 103.25) (width 0.4) (layer "F.Cu") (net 2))
 (segment (start 57.61 86.45) (end 55.2 86.45) (width 0.4) (layer "F.Cu") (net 2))
 (segment (start 43.5 102.48) (end 41.27 102.48) (width 0.4) (layer "F.Cu") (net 2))
 (segment (start 69.399 70.569) (end 70.5 71.67) (width 0.4) (layer "F.Cu") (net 2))
 (segment (start 55.2 86.45) (end 53 84.25) (width 0.4) (layer "F.Cu") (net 2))
 (segment (start 43.5 102.48) (end 46.48 102.48) (width 0.4) (layer "F.Cu") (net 2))
 (segment (start 63.181 70.569) (end 69.399 70.569) (width 0.4) (layer "F.Cu") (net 2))
 (via (at 47.25 103.25) (size 1.4) (drill 0.85) (layers "F.Cu" "B.Cu") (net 2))
 (via (at 56.25 77.5) (size 1.4) (drill 0.85) (layers "F.Cu" "B.Cu") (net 2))
 (via (at 53 84.25) (size 1.4) (drill 0.85) (layers "F.Cu" "B.Cu") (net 2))
 (segment (start 47.25 90) (end 53 84.25) (width 0.4) (layer "B.Cu") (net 2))
 (segment (start 53 84.25) (end 56.25 81) (width 0.4) (layer "B.Cu") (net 2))
 (segment (start 56.25 81) (end 56.25 77.5) (width 0.4) (layer "B.Cu") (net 2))
 (segment (start 47.25 103.25) (end 47.25 90) (width 0.4) (layer "B.Cu") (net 2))
 (segment (start 76.117214 76.75) (end 77.449 78.081786) (width 0.4) (layer "F.Cu") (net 13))
 (segment (start 76.74 88.99) (end 72.845 88.99) (width 0.4) (layer "F.Cu") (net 13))
 (segment (start 77.449 88.301) (end 76.75 89) (width 0.4) (layer "F.Cu") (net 13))
 (segment (start 77.449 78.081786) (end 77.449 88.301) (width 0.4) (layer "F.Cu") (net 13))
 (segment (start 76.75 89) (end 76.74 88.99) (width 0.4) (layer "F.Cu") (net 13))
 (segment (start 70.5 76.75) (end 76.117214 76.75) (width 0.4) (layer "F.Cu") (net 13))
 (segment (start 76.95 92.5) (end 75.38 94.07) (width 0.4) (layer "F.Cu") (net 12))
 (segment (start 65.45 79.7) (end 65.5 79.75) (width 0.4) (layer "F.Cu") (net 12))
 (segment (start 75.38 94.07) (end 72.845 94.07) (width 0.4) (layer "F.Cu") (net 12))
 (segment (start 65.45 76.75) (end 65.45 79.7) (width 0.4) (layer "F.Cu") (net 12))
 (via (at 65.5 79.75) (size 1.4) (drill 0.85) (layers "F.Cu" "B.Cu") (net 12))
 (via (at 76.95 92.5) (size 1.4) (drill 0.85) (layers "F.Cu" "B.Cu") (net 12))
 (segment (start 65.5 79.75) (end 72 79.75) (width 0.4) (layer "B.Cu") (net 12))
 (segment (start 72 79.75) (end 76.95 84.7) (width 0.4) (layer "B.Cu") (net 12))
 (segment (start 76.95 84.7) (end 76.95 92.5) (width 0.4) (layer "B.Cu") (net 12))
 (segment (start 72.845 96.61) (end 74.807 96.61) (width 0.4) (layer "F.Cu") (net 11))
 (segment (start 78.25 93.167) (end 78.25 77.75) (width 0.4) (layer "F.Cu") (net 11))
 (segment (start 74.807 96.61) (end 78.25 93.167) (width 0.4) (layer "F.Cu") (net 11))
 (segment (start 78.25 77.75) (end 74.71 74.21) (width 0.4) (layer "F.Cu") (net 11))
 (segment (start 74.71 74.21) (end 70.5 74.21) (width 0.4) (layer "F.Cu") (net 11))
 (segment (start 42.75 86.5) (end 42.75 88) (width 1) (layer "F.Cu") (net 7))
 (segment (start 43.25 86) (end 42.75 86.5) (width 1) (layer "F.Cu") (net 7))
 (segment (start 46.5 86) (end 44.5 86) (width 1) (layer "F.Cu") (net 7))
 (segment (start 49.45 97.2) (end 49.45 102) (width 1) (layer "F.Cu") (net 7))
 (segment (start 42.75 98.25) (end 42.75 96) (width 1) (layer "F.Cu") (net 7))
 (segment (start 44.5 86) (end 43.25 86) (width 1) (layer "F.Cu") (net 7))
 (segment (start 47.75 95) (end 48.5 94.25) (width 1) (layer "F.Cu") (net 7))
 (segment (start 84.4125 64.1125) (end 72.9775 64.1125) (width 1) (layer "F.Cu") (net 7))
 (segment (start 48.5 94.25) (end 48.5 88) (width 1) (layer "F.Cu") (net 7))
 (segment (start 71.8765 63.0115) (end 72.9775 64.1125) (width 1) (layer "F.Cu") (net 7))
 (segment (start 43.75 95) (end 47.75 95) (width 1) (layer "F.Cu") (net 7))
 (segment (start 44.5 86) (end 42 83.5) (width 1) (layer "F.Cu") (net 7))
 (segment (start 72.9775 64.1125) (end 70.5 66.59) (width 1) (layer "F.Cu") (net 7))
 (segment (start 47.75 95.5) (end 49.45 97.2) (width 1) (layer "F.Cu") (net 7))
 (segment (start 47.75 95) (end 47.75 95.5) (width 1) (layer "F.Cu") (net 7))
 (segment (start 42.75 96) (end 43.75 95) (width 1) (layer "F.Cu") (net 7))
 (segment (start 48.5 88) (end 46.5 86) (width 1) (layer "F.Cu") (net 7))
 (segment (start 42 83.5) (end 41.75 83.5) (width 1) (layer "F.Cu") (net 7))
 (segment (start 68.75 63.0115) (end 71.8765 63.0115) (width 1) (layer "F.Cu") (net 7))
 (via (at 41.75 83.5) (size 2) (drill 1) (layers "F.Cu" "B.Cu") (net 7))
 (via (at 68.75 63.0115) (size 2) (drill 1) (layers "F.Cu" "B.Cu") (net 7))
 (segment (start 41.75 77.25) (end 58 61) (width 1) (layer "B.Cu") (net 7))
 (segment (start 66.7385 61) (end 68.75 63.0115) (width 1) (layer "B.Cu") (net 7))
 (segment (start 58 61) (end 66.7385 61) (width 1) (layer "B.Cu") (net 7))
 (segment (start 41.75 83.5) (end 41.75 77.25) (width 1) (layer "B.Cu") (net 7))
 (segment (start 91.75 103.5) (end 84.4125 96.1625) (width 2) (layer "F.Cu") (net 4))
 (segment (start 61.59 66.59) (end 60.25 65.25) (width 1) (layer "F.Cu") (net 4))
 (segment (start 92 103.25) (end 91.75 103.5) (width 2) (layer "F.Cu") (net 4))
 (segment (start 65.45 66.59) (end 61.59 66.59) (width 1) (layer "F.Cu") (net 4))
 (segment (start 84.4125 96.1625) (end 84.4125 92.9125) (width 2) (layer "F.Cu") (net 4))
 (segment (start 84.4125 92.9125) (end 84.4625 92.9125) (width 2) (layer "F.Cu") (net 4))
 (segment (start 98 103.25) (end 92 103.25) (width 2) (layer "F.Cu") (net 4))
 (via (at 98 103.25) (size 2) (drill 1) (layers "F.Cu" "B.Cu") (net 4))
 (via (at 60.25 65.25) (size 2) (drill 1) (layers "F.Cu" "B.Cu") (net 4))
 (segment (start 62.5 65.25) (end 89.75 92.5) (width 1) (layer "B.Cu") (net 4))
 (segment (start 89.75 95) (end 98 103.25) (width 1) (layer "B.Cu") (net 4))
 (segment (start 102.5 102.25) (end 99 102.25) (width 2) (layer "B.Cu") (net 4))
 (segment (start 60.25 65.25) (end 62.5 65.25) (width 1) (layer "B.Cu") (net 4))
 (segment (start 89.75 92.5) (end 89.75 95) (width 1) (layer "B.Cu") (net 4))
 (segment (start 99 102.25) (end 98 103.25) (width 2) (layer "B.Cu") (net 4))
 (segment (start 45.75 88) (end 45.75 90.965) (width 0.4) (layer "F.Cu") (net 31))
 (segment (start 45.75 90.965) (end 45.625 91.09) (width 0.4) (layer "F.Cu") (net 31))
 (segment (start 45.75 101.155) (end 45.375 101.53) (width 0.4) (layer "F.Cu") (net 6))
 (segment (start 45.75 98.25) (end 45.75 101.155) (width 0.4) (layer "F.Cu") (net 6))
 (segment (start 41.21 92.04) (end 40.5 92.75) (width 0.4) (layer "F.Cu") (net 3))
 (segment (start 43.75 92.04) (end 41.21 92.04) (width 0.4) (layer "F.Cu") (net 3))
 (segment (start 40.5 92.75) (end 40.5 96.5) (width 0.4) (layer "F.Cu") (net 3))
 (via (at 40.5 96.5) (size 1.4) (drill 0.85) (layers "F.Cu" "B.Cu") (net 3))
 (via (at 37.5 100.5) (size 1.4) (drill 0.85) (layers "F.Cu" "B.Cu") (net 3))
 (segment (start 40.5 96.5) (end 40.5 97.5) (width 0.4) (layer "B.Cu") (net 3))
 (segment (start 40.5 97.5) (end 37.5 100.5) (width 0.4) (layer "B.Cu") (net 3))
 (segment (start 52.75 102) (end 57.3 102) (width 1.5) (layer "F.Cu") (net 19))
 (segment (start 57.3 102) (end 57.61 101.69) (width 1.5) (layer "F.Cu") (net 19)))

